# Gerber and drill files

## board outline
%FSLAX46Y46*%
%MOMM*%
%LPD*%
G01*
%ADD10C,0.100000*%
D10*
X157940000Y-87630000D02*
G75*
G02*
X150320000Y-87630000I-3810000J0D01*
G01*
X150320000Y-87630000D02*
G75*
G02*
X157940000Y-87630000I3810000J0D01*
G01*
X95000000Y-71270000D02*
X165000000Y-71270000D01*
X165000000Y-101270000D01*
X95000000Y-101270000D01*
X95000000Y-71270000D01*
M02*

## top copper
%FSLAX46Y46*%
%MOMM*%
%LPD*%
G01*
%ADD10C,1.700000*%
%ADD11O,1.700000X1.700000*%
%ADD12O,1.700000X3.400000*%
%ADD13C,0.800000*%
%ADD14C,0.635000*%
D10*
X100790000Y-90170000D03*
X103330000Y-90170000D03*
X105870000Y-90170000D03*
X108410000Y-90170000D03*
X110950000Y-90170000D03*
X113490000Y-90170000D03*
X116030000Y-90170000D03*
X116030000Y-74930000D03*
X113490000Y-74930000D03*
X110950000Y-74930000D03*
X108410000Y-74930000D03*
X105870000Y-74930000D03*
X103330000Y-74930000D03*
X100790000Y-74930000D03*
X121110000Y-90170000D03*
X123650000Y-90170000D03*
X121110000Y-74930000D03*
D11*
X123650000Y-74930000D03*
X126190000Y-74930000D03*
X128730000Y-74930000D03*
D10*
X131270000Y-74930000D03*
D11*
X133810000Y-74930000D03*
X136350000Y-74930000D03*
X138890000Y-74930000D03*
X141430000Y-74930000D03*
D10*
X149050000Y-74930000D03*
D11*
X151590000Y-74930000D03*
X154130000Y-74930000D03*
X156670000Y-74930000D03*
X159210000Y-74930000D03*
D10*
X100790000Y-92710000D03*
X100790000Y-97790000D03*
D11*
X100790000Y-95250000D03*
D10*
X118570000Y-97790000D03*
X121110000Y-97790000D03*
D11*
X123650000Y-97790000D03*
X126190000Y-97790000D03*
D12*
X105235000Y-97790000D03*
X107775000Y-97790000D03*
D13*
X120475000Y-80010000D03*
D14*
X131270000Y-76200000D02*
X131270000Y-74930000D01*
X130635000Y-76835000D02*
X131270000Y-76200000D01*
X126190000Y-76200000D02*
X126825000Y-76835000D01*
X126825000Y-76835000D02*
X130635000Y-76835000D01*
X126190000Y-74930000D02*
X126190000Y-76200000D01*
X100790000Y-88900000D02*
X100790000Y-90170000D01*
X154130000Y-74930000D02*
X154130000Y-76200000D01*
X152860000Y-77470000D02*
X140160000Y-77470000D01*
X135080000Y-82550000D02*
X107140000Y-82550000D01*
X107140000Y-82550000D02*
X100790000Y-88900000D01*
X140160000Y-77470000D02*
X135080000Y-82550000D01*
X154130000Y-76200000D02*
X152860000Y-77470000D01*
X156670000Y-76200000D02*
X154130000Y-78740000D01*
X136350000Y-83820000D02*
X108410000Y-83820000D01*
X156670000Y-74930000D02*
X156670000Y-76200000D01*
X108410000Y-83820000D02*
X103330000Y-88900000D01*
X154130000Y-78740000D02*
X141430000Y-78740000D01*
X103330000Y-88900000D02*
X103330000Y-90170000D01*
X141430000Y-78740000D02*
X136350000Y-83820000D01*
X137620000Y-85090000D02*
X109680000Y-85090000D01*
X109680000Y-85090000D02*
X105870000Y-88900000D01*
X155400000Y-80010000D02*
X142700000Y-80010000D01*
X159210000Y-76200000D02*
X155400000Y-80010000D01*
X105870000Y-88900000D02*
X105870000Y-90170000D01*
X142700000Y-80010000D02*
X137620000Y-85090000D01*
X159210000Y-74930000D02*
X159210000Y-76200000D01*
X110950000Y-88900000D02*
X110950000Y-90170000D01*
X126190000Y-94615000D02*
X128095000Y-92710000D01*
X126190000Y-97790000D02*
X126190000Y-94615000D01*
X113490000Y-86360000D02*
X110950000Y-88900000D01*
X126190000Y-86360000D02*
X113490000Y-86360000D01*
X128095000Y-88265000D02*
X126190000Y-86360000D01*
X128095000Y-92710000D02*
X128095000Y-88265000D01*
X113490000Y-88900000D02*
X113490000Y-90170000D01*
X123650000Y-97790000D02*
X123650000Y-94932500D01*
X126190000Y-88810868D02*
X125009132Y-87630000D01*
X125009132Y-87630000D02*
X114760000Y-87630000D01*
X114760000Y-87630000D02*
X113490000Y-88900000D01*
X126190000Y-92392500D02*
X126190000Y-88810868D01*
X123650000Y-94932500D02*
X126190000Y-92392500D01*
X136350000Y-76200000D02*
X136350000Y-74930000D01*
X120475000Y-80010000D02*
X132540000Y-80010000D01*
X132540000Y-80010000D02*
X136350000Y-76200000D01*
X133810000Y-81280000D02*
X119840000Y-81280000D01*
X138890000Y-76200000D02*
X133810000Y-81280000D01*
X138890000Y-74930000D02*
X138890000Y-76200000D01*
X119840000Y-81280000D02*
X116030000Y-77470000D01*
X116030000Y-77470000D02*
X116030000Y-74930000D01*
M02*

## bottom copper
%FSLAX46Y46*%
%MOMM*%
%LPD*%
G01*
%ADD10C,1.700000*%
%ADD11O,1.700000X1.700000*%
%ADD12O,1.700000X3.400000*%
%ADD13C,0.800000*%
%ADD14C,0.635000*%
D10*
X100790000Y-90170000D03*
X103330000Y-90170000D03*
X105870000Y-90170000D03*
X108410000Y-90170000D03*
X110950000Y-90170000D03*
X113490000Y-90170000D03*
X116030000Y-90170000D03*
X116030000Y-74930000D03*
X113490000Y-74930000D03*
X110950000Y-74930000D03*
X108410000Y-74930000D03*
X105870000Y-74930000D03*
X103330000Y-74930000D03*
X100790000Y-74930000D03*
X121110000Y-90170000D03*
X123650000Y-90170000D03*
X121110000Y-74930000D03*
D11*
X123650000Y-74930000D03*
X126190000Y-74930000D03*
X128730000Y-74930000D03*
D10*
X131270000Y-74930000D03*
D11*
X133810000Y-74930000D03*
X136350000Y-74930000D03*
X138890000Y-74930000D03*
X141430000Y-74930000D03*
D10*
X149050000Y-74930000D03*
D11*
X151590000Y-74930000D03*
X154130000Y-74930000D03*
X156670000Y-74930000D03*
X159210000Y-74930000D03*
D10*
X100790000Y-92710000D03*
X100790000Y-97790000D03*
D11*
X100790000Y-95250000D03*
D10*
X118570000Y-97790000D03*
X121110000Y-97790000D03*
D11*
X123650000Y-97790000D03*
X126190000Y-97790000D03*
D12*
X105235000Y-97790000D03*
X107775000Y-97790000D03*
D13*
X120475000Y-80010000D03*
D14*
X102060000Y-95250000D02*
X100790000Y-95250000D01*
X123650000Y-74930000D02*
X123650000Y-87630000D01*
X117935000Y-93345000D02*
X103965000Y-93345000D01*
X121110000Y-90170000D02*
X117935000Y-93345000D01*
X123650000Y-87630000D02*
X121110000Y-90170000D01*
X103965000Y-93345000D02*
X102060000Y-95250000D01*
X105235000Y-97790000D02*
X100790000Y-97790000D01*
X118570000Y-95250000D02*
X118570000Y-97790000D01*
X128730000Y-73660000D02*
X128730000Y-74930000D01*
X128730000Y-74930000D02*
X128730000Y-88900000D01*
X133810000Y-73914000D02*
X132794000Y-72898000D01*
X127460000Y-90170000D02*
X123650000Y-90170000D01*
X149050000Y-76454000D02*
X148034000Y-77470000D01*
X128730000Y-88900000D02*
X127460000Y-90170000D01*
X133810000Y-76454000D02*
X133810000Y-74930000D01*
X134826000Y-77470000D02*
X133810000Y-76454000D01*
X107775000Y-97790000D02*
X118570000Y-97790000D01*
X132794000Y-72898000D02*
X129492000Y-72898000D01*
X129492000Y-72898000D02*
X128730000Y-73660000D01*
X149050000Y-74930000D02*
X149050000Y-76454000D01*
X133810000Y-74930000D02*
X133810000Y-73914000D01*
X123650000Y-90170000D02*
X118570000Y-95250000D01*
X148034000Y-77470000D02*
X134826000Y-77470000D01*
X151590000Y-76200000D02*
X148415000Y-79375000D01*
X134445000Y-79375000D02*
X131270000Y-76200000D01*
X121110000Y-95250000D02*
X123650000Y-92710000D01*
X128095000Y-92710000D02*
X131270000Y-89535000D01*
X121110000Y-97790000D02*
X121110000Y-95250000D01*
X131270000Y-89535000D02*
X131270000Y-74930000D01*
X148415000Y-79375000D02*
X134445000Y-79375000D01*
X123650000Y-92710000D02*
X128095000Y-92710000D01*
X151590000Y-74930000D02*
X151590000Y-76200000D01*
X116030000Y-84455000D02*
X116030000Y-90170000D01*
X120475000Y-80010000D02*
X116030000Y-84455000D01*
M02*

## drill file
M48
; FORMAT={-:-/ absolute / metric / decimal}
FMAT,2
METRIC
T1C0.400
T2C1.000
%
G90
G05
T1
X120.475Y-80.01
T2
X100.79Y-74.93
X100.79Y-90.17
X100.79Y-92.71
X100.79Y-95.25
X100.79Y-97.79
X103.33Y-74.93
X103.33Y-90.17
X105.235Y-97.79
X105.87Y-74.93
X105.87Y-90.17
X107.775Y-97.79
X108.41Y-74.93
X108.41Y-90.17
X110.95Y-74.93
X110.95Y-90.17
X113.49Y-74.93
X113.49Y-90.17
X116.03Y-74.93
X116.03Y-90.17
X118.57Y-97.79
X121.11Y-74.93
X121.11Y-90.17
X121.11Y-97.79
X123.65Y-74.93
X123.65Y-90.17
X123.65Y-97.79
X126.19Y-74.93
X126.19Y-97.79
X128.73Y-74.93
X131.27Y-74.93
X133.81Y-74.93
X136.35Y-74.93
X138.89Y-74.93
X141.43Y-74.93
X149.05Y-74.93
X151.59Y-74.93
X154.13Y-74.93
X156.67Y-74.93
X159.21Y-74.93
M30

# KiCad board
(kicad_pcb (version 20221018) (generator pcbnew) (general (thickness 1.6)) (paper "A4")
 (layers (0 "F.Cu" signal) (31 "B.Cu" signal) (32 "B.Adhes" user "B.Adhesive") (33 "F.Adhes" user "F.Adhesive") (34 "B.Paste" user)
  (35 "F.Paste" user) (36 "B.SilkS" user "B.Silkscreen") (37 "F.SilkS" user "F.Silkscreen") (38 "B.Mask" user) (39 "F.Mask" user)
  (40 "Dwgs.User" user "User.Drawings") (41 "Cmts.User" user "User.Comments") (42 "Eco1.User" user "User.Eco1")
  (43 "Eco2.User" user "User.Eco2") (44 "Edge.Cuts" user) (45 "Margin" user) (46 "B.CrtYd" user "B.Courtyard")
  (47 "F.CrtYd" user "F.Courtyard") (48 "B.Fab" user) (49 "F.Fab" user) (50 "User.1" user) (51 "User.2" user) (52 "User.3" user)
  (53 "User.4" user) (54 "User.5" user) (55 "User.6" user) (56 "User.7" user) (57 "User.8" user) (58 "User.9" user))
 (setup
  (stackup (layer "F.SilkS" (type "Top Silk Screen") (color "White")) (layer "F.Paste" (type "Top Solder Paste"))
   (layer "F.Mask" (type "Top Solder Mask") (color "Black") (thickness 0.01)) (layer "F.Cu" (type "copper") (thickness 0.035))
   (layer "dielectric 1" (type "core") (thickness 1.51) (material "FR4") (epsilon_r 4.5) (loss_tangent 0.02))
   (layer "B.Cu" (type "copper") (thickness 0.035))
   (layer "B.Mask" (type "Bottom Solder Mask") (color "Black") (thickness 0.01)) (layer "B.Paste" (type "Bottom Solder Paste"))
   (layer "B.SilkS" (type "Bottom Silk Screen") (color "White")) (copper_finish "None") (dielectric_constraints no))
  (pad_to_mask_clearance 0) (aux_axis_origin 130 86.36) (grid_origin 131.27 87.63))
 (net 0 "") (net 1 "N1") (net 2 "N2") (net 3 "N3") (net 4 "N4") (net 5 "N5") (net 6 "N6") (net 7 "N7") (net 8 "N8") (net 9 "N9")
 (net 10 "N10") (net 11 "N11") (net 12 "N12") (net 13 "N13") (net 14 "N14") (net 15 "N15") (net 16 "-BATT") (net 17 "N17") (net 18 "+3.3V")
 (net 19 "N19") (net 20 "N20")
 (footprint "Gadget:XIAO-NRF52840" (layer "F.Cu") (at 108.41 82.55 90)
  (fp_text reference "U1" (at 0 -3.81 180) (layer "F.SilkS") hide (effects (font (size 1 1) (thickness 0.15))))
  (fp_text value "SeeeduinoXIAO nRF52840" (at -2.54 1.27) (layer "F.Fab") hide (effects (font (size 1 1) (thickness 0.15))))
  (pad "1" thru_hole circle (at -7.62 -7.62 90) (size 1.7 1.7) (drill 1) (layers "*.Cu" "*.Mask") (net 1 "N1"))
  (pad "2" thru_hole circle (at -7.62 -5.08 90) (size 1.7 1.7) (drill 1) (layers "*.Cu" "*.Mask") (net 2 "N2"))
  (pad "3" thru_hole circle (at -7.62 -2.54 90) (size 1.7 1.7) (drill 1) (layers "*.Cu" "*.Mask") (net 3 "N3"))
  (pad "4" thru_hole circle (at -7.62 0 90) (size 1.7 1.7) (drill 1) (layers "*.Cu" "*.Mask") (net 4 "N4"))
  (pad "5" thru_hole circle (at -7.62 2.54 90) (size 1.7 1.7) (drill 1) (layers "*.Cu" "*.Mask") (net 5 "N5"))
  (pad "6" thru_hole circle (at -7.62 5.08 90) (size 1.7 1.7) (drill 1) (layers "*.Cu" "*.Mask") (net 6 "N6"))
  (pad "7" thru_hole circle (at -7.62 7.62 90) (size 1.7 1.7) (drill 1) (layers "*.Cu" "*.Mask") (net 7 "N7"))
  (pad "8" thru_hole circle (at 7.62 7.62 90) (size 1.7 1.7) (drill 1) (layers "*.Cu" "*.Mask") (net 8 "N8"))
  (pad "9" thru_hole circle (at 7.62 5.08 90) (size 1.7 1.7) (drill 1) (layers "*.Cu" "*.Mask") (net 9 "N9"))
  (pad "10" thru_hole circle (at 7.62 2.54 90) (size 1.7 1.7) (drill 1) (layers "*.Cu" "*.Mask") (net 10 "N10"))
  (pad "11" thru_hole circle (at 7.62 0 90) (size 1.7 1.7) (drill 1) (layers "*.Cu" "*.Mask") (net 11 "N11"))
  (pad "12" thru_hole circle (at 7.62 -2.54 90) (size 1.7 1.7) (drill 1) (layers "*.Cu" "*.Mask") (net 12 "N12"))
  (pad "13" thru_hole circle (at 7.62 -5.08 90) (size 1.7 1.7) (drill 1) (layers "*.Cu" "*.Mask") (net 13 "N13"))
  (pad "14" thru_hole circle (at 7.62 -7.62 90) (size 1.7 1.7) (drill 1) (layers "*.Cu" "*.Mask") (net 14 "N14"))
  (pad "15" thru_hole circle (at -7.62 12.7 270) (size 1.7 1.7) (drill 1) (layers "*.Cu" "*.Mask") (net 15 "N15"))
  (pad "16" thru_hole circle (at -7.62 15.24 270) (size 1.7 1.7) (drill 1) (layers "*.Cu" "*.Mask") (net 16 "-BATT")))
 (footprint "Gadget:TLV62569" (layer "F.Cu") (at 124.92 74.93 90)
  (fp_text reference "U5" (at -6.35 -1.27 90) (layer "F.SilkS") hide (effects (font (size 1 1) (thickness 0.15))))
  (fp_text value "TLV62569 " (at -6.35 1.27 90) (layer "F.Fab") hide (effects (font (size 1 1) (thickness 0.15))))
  (pad "1" thru_hole circle (at 0 -3.81 90) (size 1.7 1.7) (drill 1) (layers "*.Cu" "*.Mask") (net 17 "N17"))
  (pad "2" thru_hole oval (at 0 -1.27 90) (size 1.7 1.7) (drill 1) (layers "*.Cu" "*.Mask") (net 15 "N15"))
  (pad "3" thru_hole oval (at 0 1.27 90) (size 1.7 1.7) (drill 1) (layers "*.Cu" "*.Mask") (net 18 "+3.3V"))
  (pad "4" thru_hole oval (at 0 3.81 90) (size 1.7 1.7) (drill 1) (layers "*.Cu" "*.Mask") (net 16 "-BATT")))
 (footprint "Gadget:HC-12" (layer "F.Cu") (at 136.35 74.93 90)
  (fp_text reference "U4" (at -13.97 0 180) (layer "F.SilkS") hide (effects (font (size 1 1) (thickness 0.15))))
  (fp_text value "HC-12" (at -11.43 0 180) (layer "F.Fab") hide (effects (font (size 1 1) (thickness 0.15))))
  (pad "1" thru_hole circle (at 0 -5.08 90) (size 1.7 1.7) (drill 1) (layers "*.Cu" "*.Mask") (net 18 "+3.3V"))
  (pad "2" thru_hole oval (at 0 -2.54 90) (size 1.7 1.7) (drill 1) (layers "*.Cu" "*.Mask") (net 16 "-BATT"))
  (pad "3" thru_hole oval (at 0 0 90) (size 1.7 1.7) (drill 1) (layers "*.Cu" "*.Mask") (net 7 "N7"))
  (pad "4" thru_hole oval (at 0 2.54 90) (size 1.7 1.7) (drill 1) (layers "*.Cu" "*.Mask") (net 8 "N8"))
  (pad "5" thru_hole oval (at 0 5.08 90) (size 1.7 1.7) (drill 1) (layers "*.Cu" "*.Mask") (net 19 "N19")))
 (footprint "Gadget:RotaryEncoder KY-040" (layer "F.Cu") (at 151.59 74.93 90)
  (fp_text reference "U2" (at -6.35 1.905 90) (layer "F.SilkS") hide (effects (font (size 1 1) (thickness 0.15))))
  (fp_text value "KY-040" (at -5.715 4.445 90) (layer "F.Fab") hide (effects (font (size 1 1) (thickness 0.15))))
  (pad "1" thru_hole circle (at 0 -2.54 90) (size 1.7 1.7) (drill 1) (layers "*.Cu" "*.Mask") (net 16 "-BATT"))
  (pad "2" thru_hole oval (at 0 0 90) (size 1.7 1.7) (drill 1) (layers "*.Cu" "*.Mask") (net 18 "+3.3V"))
  (pad "3" thru_hole oval (at 0 2.54 90) (size 1.7 1.7) (drill 1) (layers "*.Cu" "*.Mask") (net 1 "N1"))
  (pad "4" thru_hole oval (at 0 5.08 90) (size 1.7 1.7) (drill 1) (layers "*.Cu" "*.Mask") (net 2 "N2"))
  (pad "5" thru_hole oval (at 0 7.62 90) (size 1.7 1.7) (drill 1) (layers "*.Cu" "*.Mask") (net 3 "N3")))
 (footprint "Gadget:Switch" (layer "F.Cu") (at 100.79 97.79 180)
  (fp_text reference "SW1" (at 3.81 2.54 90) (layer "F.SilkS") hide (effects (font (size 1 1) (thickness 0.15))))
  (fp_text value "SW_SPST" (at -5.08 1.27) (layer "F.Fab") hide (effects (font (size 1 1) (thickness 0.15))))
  (pad "" thru_hole circle (at 0 5.08 180) (size 1.7 1.7) (drill 1) (layers "*.Cu" "*.Mask"))
  (pad "1" thru_hole circle (at 0 0 180) (size 1.7 1.7) (drill 1) (layers "*.Cu" "*.Mask") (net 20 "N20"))
  (pad "2" thru_hole oval (at 0 2.54 180) (size 1.7 1.7) (drill 1) (layers "*.Cu" "*.Mask") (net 15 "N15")))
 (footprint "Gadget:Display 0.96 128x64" (layer "B.Cu") (at 122.38 97.79 -90)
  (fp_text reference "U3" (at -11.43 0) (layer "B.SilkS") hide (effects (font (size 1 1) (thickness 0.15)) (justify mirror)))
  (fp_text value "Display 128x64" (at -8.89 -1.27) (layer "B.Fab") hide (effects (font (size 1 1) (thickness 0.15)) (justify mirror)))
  (pad "1" thru_hole circle (at 0 3.81 270) (size 1.7 1.7) (drill 1) (layers "*.Cu" "*.Mask") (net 16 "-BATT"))
  (pad "2" thru_hole circle (at 0 1.27 270) (size 1.7 1.7) (drill 1) (layers "*.Cu" "*.Mask") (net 18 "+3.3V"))
  (pad "3" thru_hole oval (at 0 -1.27 270) (size 1.7 1.7) (drill 1) (layers "*.Cu" "*.Mask") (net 6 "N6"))
  (pad "4" thru_hole oval (at 0 -3.81 270) (size 1.7 1.7) (drill 1) (layers "*.Cu" "*.Mask") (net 5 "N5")))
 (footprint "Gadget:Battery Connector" (layer "B.Cu") (at 105.235 97.79 -90)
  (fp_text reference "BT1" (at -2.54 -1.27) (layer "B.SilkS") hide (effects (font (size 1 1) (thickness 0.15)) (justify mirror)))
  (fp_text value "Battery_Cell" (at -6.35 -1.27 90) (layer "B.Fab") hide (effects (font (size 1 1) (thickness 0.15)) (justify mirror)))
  (pad "1" thru_hole oval (at 0 0 270) (size 3.4 1.7) (drill 1) (layers "*.Cu" "*.Mask") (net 20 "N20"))
  (pad "2" thru_hole oval (at 0 -2.54 270) (size 3.4 1.7) (drill 1) (layers "*.Cu" "*.Mask") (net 16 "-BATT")))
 (gr_circle (center 154.13 87.63) (end 157.94 87.63) (stroke (width 0.1) (type default)) (fill none) (layer "Edge.Cuts"))
 (gr_rect (start 95 71.27) (end 165 101.27) (stroke (width 0.1) (type default)) (fill none) (layer "Edge.Cuts"))
 (segment (start 102.06 95.25) (end 100.79 95.25) (width 0.635) (layer "B.Cu") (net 15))
 (segment (start 123.65 74.93) (end 123.65 87.63) (width 0.635) (layer "B.Cu") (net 15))
 (segment (start 117.935 93.345) (end 103.965 93.345) (width 0.635) (layer "B.Cu") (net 15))
 (segment (start 121.11 90.17) (end 117.935 93.345) (width 0.635) (layer "B.Cu") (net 15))
 (segment (start 123.65 87.63) (end 121.11 90.17) (width 0.635) (layer "B.Cu") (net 15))
 (segment (start 103.965 93.345) (end 102.06 95.25) (width 0.635) (layer "B.Cu") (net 15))
 (segment (start 105.235 97.79) (end 100.79 97.79) (width 0.635) (layer "B.Cu") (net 20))
 (segment (start 118.57 95.25) (end 118.57 97.79) (width 0.635) (layer "B.Cu") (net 16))
 (segment (start 128.73 73.66) (end 128.73 74.93) (width 0.635) (layer "B.Cu") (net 16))
 (segment (start 128.73 74.93) (end 128.73 88.9) (width 0.635) (layer "B.Cu") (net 16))
 (segment (start 133.81 73.914) (end 132.794 72.898) (width 0.635) (layer "B.Cu") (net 16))
 (segment (start 127.46 90.17) (end 123.65 90.17) (width 0.635) (layer "B.Cu") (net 16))
 (segment (start 149.05 76.454) (end 148.034 77.47) (width 0.635) (layer "B.Cu") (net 16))
 (segment (start 128.73 88.9) (end 127.46 90.17) (width 0.635) (layer "B.Cu") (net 16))
 (segment (start 133.81 76.454) (end 133.81 74.93) (width 0.635) (layer "B.Cu") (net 16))
 (segment (start 134.826 77.47) (end 133.81 76.454) (width 0.635) (layer "B.Cu") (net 16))
 (segment (start 107.775 97.79) (end 118.57 97.79) (width 0.635) (layer "B.Cu") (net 16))
 (segment (start 132.794 72.898) (end 129.492 72.898) (width 0.635) (layer "B.Cu") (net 16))
 (segment (start 129.492 72.898) (end 128.73 73.66) (width 0.635) (layer "B.Cu") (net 16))
 (segment (start 149.05 74.93) (end 149.05 76.454) (width 0.635) (layer "B.Cu") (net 16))
 (segment (start 133.81 74.93) (end 133.81 73.914) (width 0.635) (layer "B.Cu") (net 16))
 (segment (start 123.65 90.17) (end 118.57 95.25) (width 0.635) (layer "B.Cu") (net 16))
 (segment (start 148.034 77.47) (end 134.826 77.47) (width 0.635) (layer "B.Cu") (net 16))
 (segment (start 131.27 76.2) (end 131.27 74.93) (width 0.635) (layer "F.Cu") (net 18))
 (segment (start 130.635 76.835) (end 131.27 76.2) (width 0.635) (layer "F.Cu") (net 18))
 (segment (start 126.19 76.2) (end 126.825 76.835) (width 0.635) (layer "F.Cu") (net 18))
 (segment (start 126.825 76.835) (end 130.635 76.835) (width 0.635) (layer "F.Cu") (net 18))
 (segment (start 126.19 74.93) (end 126.19 76.2) (width 0.635) (layer "F.Cu") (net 18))
 (segment (start 151.59 76.2) (end 148.415 79.375) (width 0.635) (layer "B.Cu") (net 18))
 (segment (start 134.445 79.375) (end 131.27 76.2) (width 0.635) (layer "B.Cu") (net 18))
 (segment (start 121.11 95.25) (end 123.65 92.71) (width 0.635) (layer "B.Cu") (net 18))
 (segment (start 128.095 92.71) (end 131.27 89.535) (width 0.635) (layer "B.Cu") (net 18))
 (segment (start 121.11 97.79) (end 121.11 95.25) (width 0.635) (layer "B.Cu") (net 18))
 (segment (start 131.27 89.535) (end 131.27 74.93) (width 0.635) (layer "B.Cu") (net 18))
 (segment (start 148.415 79.375) (end 134.445 79.375) (width 0.635) (layer "B.Cu") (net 18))
 (segment (start 123.65 92.71) (end 128.095 92.71) (width 0.635) (layer "B.Cu") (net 18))
 (segment (start 151.59 74.93) (end 151.59 76.2) (width 0.635) (layer "B.Cu") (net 18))
 (segment (start 100.79 88.9) (end 100.79 90.17) (width 0.635) (layer "F.Cu") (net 1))
 (segment (start 154.13 74.93) (end 154.13 76.2) (width 0.635) (layer "F.Cu") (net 1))
 (segment (start 152.86 77.47) (end 140.16 77.47) (width 0.635) (layer "F.Cu") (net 1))
 (segment (start 135.08 82.55) (end 107.14 82.55) (width 0.635) (layer "F.Cu") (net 1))
 (segment (start 107.14 82.55) (end 100.79 88.9) (width 0.635) (layer "F.Cu") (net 1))
 (segment (start 140.16 77.47) (end 135.08 82.55) (width 0.635) (layer "F.Cu") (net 1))
 (segment (start 154.13 76.2) (end 152.86 77.47) (width 0.635) (layer "F.Cu") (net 1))
 (segment (start 156.67 76.2) (end 154.13 78.74) (width 0.635) (layer "F.Cu") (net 2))
 (segment (start 136.35 83.82) (end 108.41 83.82) (width 0.635) (layer "F.Cu") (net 2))
 (segment (start 156.67 74.93) (end 156.67 76.2) (width 0.635) (layer "F.Cu") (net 2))
 (segment (start 108.41 83.82) (end 103.33 88.9) (width 0.635) (layer "F.Cu") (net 2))
 (segment (start 154.13 78.74) (end 141.43 78.74) (width 0.635) (layer "F.Cu") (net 2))
 (segment (start 103.33 88.9) (end 103.33 90.17) (width 0.635) (layer "F.Cu") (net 2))
 (segment (start 141.43 78.74) (end 136.35 83.82) (width 0.635) (layer "F.Cu") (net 2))
 (segment (start 137.62 85.09) (end 109.68 85.09) (width 0.635) (layer "F.Cu") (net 3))
 (segment (start 109.68 85.09) (end 105.87 88.9) (width 0.635) (layer "F.Cu") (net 3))
 (segment (start 155.4 80.01) (end 142.7 80.01) (width 0.635) (layer "F.Cu") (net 3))
 (segment (start 159.21 76.2) (end 155.4 80.01) (width 0.635) (layer "F.Cu") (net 3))
 (segment (start 105.87 88.9) (end 105.87 90.17) (width 0.635) (layer "F.Cu") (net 3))
 (segment (start 142.7 80.01) (end 137.62 85.09) (width 0.635) (layer "F.Cu") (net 3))
 (segment (start 159.21 74.93) (end 159.21 76.2) (width 0.635) (layer "F.Cu") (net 3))
 (segment (start 110.95 88.9) (end 110.95 90.17) (width 0.635) (layer "F.Cu") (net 5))
 (segment (start 126.19 94.615) (end 128.095 92.71) (width 0.635) (layer "F.Cu") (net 5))
 (segment (start 126.19 97.79) (end 126.19 94.615) (width 0.635) (layer "F.Cu") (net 5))
 (segment (start 113.49 86.36) (end 110.95 88.9) (width 0.635) (layer "F.Cu") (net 5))
 (segment (start 126.19 86.36) (end 113.49 86.36) (width 0.635) (layer "F.Cu") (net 5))
 (segment (start 128.095 88.265) (end 126.19 86.36) (width 0.635) (layer "F.Cu") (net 5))
 (segment (start 128.095 92.71) (end 128.095 88.265) (width 0.635) (layer "F.Cu") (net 5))
 (segment (start 113.49 88.9) (end 113.49 90.17) (width 0.635) (layer "F.Cu") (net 6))
 (segment (start 123.65 97.79) (end 123.65 94.9325) (width 0.635) (layer "F.Cu") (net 6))
 (segment (start 126.19 88.810868) (end 125.009132 87.63) (width 0.635) (layer "F.Cu") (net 6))
 (segment (start 125.009132 87.63) (end 114.76 87.63) (width 0.635) (layer "F.Cu") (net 6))
 (segment (start 114.76 87.63) (end 113.49 88.9) (width 0.635) (layer "F.Cu") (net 6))
 (segment (start 126.19 92.3925) (end 126.19 88.810868) (width 0.635) (layer "F.Cu") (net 6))
 (segment (start 123.65 94.9325) (end 126.19 92.3925) (width 0.635) (layer "F.Cu") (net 6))
 (segment (start 136.35 76.2) (end 136.35 74.93) (width 0.635) (layer "F.Cu") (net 7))
 (segment (start 120.475 80.01) (end 132.54 80.01) (width 0.635) (layer "F.Cu") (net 7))
 (segment (start 132.54 80.01) (end 136.35 76.2) (width 0.635) (layer "F.Cu") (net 7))
 (via (at 120.475 80.01) (size 0.8) (drill 0.4) (layers "F.Cu" "B.Cu") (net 7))
 (segment (start 116.03 84.455) (end 116.03 90.17) (width 0.635) (layer "B.Cu") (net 7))
 (segment (start 120.475 80.01) (end 116.03 84.455) (width 0.635) (layer "B.Cu") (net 7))
 (segment (start 133.81 81.28) (end 119.84 81.28) (width 0.635) (layer "F.Cu") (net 8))
 (segment (start 138.89 76.2) (end 133.81 81.28) (width 0.635) (layer "F.Cu") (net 8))
 (segment (start 138.89 74.93) (end 138.89 76.2) (width 0.635) (layer "F.Cu") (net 8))
 (segment (start 119.84 81.28) (end 116.03 77.47) (width 0.635) (layer "F.Cu") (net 8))
 (segment (start 116.03 77.47) (end 116.03 74.93) (width 0.635) (layer "F.Cu") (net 8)))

